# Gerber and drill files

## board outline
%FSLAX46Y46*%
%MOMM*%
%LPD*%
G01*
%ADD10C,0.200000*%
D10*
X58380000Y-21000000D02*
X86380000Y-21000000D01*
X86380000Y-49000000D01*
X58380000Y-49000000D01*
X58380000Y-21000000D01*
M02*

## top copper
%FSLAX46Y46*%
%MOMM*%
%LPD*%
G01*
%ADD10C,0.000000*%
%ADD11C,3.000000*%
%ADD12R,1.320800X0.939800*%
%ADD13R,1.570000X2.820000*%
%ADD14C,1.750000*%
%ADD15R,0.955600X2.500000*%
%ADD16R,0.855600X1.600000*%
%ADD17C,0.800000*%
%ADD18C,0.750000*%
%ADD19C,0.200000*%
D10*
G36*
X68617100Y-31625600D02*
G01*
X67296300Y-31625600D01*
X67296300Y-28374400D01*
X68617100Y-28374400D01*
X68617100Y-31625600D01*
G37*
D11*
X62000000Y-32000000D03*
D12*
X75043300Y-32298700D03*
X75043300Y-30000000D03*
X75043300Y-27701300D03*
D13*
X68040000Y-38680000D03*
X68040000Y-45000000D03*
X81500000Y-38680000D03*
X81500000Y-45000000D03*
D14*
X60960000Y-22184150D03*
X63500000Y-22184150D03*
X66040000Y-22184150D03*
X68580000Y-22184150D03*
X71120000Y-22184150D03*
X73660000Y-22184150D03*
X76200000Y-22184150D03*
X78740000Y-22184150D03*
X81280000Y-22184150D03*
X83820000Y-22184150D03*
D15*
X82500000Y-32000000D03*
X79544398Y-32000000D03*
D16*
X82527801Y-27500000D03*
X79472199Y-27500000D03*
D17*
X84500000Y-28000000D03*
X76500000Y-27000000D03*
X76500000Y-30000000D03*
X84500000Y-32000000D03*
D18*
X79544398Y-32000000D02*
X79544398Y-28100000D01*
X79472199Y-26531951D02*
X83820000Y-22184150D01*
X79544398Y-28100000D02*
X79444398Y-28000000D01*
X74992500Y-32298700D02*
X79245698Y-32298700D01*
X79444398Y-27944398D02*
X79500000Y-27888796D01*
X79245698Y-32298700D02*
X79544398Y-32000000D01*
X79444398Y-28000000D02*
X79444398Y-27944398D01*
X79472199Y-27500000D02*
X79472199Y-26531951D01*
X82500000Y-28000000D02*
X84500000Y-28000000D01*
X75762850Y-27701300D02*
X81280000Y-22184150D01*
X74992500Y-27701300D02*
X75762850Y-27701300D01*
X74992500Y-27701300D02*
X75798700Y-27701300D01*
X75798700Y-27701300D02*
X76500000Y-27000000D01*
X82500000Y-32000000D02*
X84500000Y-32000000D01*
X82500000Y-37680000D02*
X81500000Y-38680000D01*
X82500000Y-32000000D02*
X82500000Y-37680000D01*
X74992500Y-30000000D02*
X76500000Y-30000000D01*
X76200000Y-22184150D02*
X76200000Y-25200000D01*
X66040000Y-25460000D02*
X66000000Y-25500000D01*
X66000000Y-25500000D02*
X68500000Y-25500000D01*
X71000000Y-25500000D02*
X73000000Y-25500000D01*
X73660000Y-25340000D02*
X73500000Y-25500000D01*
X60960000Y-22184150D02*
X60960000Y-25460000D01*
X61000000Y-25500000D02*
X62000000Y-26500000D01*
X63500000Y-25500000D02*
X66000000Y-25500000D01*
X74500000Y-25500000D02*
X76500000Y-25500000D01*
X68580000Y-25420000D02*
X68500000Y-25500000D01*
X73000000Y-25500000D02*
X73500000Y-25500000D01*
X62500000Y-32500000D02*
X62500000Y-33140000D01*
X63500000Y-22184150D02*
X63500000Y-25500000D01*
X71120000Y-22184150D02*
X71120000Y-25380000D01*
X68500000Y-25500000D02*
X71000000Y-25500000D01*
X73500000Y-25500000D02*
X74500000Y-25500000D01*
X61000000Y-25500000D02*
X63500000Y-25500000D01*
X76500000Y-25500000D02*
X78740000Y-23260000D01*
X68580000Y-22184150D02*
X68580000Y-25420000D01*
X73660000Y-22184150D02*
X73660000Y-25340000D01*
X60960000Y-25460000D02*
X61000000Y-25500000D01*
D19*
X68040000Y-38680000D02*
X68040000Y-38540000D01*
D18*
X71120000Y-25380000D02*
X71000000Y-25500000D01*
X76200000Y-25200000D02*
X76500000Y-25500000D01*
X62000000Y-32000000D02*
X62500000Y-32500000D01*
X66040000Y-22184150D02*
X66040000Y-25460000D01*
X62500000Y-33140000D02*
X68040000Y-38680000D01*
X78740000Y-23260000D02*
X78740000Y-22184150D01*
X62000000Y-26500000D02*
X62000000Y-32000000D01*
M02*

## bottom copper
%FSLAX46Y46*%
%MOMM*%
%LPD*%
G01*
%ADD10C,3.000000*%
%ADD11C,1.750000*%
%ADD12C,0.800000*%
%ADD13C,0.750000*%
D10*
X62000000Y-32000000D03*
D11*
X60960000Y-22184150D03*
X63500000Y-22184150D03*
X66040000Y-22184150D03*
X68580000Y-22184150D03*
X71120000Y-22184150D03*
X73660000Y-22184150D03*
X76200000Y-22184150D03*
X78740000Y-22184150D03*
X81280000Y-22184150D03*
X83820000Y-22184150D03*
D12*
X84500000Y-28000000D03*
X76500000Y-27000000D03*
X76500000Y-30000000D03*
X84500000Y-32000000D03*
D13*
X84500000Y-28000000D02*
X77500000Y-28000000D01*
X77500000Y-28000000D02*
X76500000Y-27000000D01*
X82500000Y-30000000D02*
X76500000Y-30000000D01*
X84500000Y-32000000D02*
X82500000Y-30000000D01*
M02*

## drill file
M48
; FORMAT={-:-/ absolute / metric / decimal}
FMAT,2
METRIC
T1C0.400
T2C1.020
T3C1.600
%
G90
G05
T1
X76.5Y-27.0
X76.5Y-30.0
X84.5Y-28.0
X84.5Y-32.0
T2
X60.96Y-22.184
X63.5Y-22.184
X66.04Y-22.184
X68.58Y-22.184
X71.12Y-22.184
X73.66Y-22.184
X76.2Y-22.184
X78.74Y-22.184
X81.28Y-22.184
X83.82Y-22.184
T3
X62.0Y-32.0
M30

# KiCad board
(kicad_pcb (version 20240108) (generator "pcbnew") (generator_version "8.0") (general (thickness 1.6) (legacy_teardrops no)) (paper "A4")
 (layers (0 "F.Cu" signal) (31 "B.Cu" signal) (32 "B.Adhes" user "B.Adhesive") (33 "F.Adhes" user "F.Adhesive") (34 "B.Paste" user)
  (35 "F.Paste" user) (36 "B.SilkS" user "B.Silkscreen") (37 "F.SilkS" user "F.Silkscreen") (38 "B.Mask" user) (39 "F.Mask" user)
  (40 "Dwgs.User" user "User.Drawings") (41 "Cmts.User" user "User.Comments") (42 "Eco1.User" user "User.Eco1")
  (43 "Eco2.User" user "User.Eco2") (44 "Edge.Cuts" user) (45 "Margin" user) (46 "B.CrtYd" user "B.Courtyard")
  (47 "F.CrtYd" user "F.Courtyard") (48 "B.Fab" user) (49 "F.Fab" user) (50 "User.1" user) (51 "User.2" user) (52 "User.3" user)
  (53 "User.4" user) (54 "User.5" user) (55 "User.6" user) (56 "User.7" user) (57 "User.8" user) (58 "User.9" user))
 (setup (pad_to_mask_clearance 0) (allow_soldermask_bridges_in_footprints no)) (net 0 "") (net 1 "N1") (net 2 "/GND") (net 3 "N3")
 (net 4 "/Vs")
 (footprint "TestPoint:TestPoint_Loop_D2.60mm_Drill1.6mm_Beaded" (layer "F.Cu") (at 62 32)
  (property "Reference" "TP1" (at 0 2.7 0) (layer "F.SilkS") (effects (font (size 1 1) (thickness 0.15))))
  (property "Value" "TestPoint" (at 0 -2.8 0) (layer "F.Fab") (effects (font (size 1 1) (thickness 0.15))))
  (pad "1" thru_hole circle (at 0 0) (size 3 3) (drill 1.6) (layers "*.Cu" "*.Mask") (remove_unused_layers no) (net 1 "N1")))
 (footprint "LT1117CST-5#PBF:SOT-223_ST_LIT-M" (layer "F.Cu") (at 71.5 30 90)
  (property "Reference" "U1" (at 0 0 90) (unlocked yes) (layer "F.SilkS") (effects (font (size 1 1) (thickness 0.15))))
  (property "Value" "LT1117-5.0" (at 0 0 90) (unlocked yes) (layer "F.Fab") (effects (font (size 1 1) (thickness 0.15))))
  (fp_poly
   (pts (xy 1.6256 -4.2037) (xy -1.6256 -4.2037) (xy -1.6256 -2.8829) (xy 1.6256 -2.8829)) (stroke (width 0) (type solid)) (fill solid)
   (layer "F.Cu"))
  (pad "1" smd rect (at -2.2987 3.5433 90) (size 0.9398 1.3208) (layers "F.Cu" "F.Paste" "F.Mask") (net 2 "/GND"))
  (pad "2" smd rect (at 0 3.5433 90) (size 0.9398 1.3208) (layers "F.Cu" "F.Paste" "F.Mask") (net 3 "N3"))
  (pad "3" smd rect (at 2.2987 3.5433 90) (size 0.9398 1.3208) (layers "F.Cu" "F.Paste" "F.Mask") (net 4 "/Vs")))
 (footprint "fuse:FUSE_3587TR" (layer "F.Cu") (at 74.77 41.84)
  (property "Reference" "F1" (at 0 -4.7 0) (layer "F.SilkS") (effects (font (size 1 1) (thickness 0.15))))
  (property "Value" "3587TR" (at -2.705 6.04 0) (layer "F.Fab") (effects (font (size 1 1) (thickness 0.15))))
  (pad "1_1" smd rect (at -6.73 -3.16) (size 1.57 2.82) (layers "F.Cu" "F.Paste" "F.Mask") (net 1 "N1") (solder_mask_margin 0.102))
  (pad "1_2" smd rect (at -6.73 3.16) (size 1.57 2.82) (layers "F.Cu" "F.Paste" "F.Mask") (solder_mask_margin 0.102))
  (pad "2_1" smd rect (at 6.73 -3.16) (size 1.57 2.82) (layers "F.Cu" "F.Paste" "F.Mask") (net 3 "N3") (solder_mask_margin 0.102))
  (pad "2_2" smd rect (at 6.73 3.16) (size 1.57 2.82) (layers "F.Cu" "F.Paste" "F.Mask") (solder_mask_margin 0.102)))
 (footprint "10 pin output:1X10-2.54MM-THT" (layer "F.Cu") (at 60.96 22.18415)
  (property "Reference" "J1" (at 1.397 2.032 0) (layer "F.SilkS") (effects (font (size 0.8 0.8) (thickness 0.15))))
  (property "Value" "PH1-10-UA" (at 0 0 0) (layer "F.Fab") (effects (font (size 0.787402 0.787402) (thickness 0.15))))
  (pad "1" thru_hole circle (at 0 0) (size 1.75 1.75) (drill 1.02) (layers "*.Cu" "*.Mask") (remove_unused_layers no) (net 1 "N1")
   (solder_mask_margin 0.102))
  (pad "2" thru_hole circle (at 2.54 0) (size 1.75 1.75) (drill 1.02) (layers "*.Cu" "*.Mask") (remove_unused_layers no) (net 1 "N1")
   (solder_mask_margin 0.102))
  (pad "3" thru_hole circle (at 5.08 0) (size 1.75 1.75) (drill 1.02) (layers "*.Cu" "*.Mask") (remove_unused_layers no) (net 1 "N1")
   (solder_mask_margin 0.102))
  (pad "4" thru_hole circle (at 7.62 0) (size 1.75 1.75) (drill 1.02) (layers "*.Cu" "*.Mask") (remove_unused_layers no) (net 1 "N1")
   (solder_mask_margin 0.102))
  (pad "5" thru_hole circle (at 10.16 0) (size 1.75 1.75) (drill 1.02) (layers "*.Cu" "*.Mask") (remove_unused_layers no) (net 1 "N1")
   (solder_mask_margin 0.102))
  (pad "6" thru_hole circle (at 12.7 0) (size 1.75 1.75) (drill 1.02) (layers "*.Cu" "*.Mask") (remove_unused_layers no) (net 1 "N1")
   (solder_mask_margin 0.102))
  (pad "7" thru_hole circle (at 15.24 0) (size 1.75 1.75) (drill 1.02) (layers "*.Cu" "*.Mask") (remove_unused_layers no) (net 1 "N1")
   (solder_mask_margin 0.102))
  (pad "8" thru_hole circle (at 17.78 0) (size 1.75 1.75) (drill 1.02) (layers "*.Cu" "*.Mask") (remove_unused_layers no) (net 1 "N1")
   (solder_mask_margin 0.102))
  (pad "9" thru_hole circle (at 20.32 0) (size 1.75 1.75) (drill 1.02) (layers "*.Cu" "*.Mask") (remove_unused_layers no) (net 4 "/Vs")
   (solder_mask_margin 0.102))
  (pad "10" thru_hole circle (at 22.86 0) (size 1.75 1.75) (drill 1.02) (layers "*.Cu" "*.Mask") (remove_unused_layers no) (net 2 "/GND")
   (solder_mask_margin 0.102)))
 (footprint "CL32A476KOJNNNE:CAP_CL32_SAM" (layer "F.Cu") (at 81.022199 32 180)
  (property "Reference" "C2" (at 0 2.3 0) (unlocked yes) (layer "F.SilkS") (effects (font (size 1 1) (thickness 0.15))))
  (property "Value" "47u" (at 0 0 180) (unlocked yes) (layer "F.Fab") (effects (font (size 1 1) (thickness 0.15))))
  (pad "1" smd rect (at -1.477801 0 180) (size 0.9556 2.5) (layers "F.Cu" "F.Paste" "F.Mask") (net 3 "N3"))
  (pad "2" smd rect (at 1.477801 0 180) (size 0.9556 2.5) (layers "F.Cu" "F.Paste" "F.Mask") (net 2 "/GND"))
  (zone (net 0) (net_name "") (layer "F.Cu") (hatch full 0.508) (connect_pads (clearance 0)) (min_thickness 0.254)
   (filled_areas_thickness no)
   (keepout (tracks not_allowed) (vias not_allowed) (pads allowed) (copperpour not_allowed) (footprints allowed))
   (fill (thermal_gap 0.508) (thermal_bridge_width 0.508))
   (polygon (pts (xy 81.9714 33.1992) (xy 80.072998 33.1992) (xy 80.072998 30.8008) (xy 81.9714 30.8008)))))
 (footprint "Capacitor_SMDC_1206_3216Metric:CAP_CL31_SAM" (layer "F.Cu") (at 81 27.5 180)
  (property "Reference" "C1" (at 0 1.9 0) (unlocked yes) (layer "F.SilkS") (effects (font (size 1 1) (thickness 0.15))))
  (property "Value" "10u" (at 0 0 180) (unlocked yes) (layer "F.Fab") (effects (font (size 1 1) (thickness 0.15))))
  (pad "1" smd rect (at -1.527801 0 180) (size 0.8556 1.6) (layers "F.Cu" "F.Paste" "F.Mask") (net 4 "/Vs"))
  (pad "2" smd rect (at 1.527801 0 180) (size 0.8556 1.6) (layers "F.Cu" "F.Paste" "F.Mask") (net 2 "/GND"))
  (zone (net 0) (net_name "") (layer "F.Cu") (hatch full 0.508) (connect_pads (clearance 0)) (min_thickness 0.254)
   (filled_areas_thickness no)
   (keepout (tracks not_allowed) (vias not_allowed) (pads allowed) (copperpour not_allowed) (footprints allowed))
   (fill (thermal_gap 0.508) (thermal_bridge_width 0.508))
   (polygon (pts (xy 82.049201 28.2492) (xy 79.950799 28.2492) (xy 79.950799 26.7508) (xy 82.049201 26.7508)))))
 (gr_rect (start 58.38 21) (end 86.38 49) (stroke (width 0.2) (type default)) (fill none) (layer "Edge.Cuts"))
 (segment (start 79.544398 32) (end 79.544398 28.1) (width 0.75) (layer "F.Cu") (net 2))
 (segment (start 79.472199 26.531951) (end 83.82 22.18415) (width 0.75) (layer "F.Cu") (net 2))
 (segment (start 79.544398 28.1) (end 79.444398 28) (width 0.75) (layer "F.Cu") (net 2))
 (segment (start 74.9925 32.2987) (end 79.245698 32.2987) (width 0.75) (layer "F.Cu") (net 2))
 (segment (start 79.444398 27.944398) (end 79.5 27.888796) (width 0.75) (layer "F.Cu") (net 2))
 (segment (start 79.245698 32.2987) (end 79.544398 32) (width 0.75) (layer "F.Cu") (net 2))
 (segment (start 79.444398 28) (end 79.444398 27.944398) (width 0.75) (layer "F.Cu") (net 2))
 (segment (start 79.472199 27.5) (end 79.472199 26.531951) (width 0.75) (layer "F.Cu") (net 2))
 (segment (start 82.5 28) (end 84.5 28) (width 0.75) (layer "F.Cu") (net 4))
 (segment (start 75.76285 27.7013) (end 81.28 22.18415) (width 0.75) (layer "F.Cu") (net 4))
 (segment (start 74.9925 27.7013) (end 75.76285 27.7013) (width 0.75) (layer "F.Cu") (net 4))
 (segment (start 74.9925 27.7013) (end 75.7987 27.7013) (width 0.75) (layer "F.Cu") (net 4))
 (segment (start 75.7987 27.7013) (end 76.5 27) (width 0.75) (layer "F.Cu") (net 4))
 (via (at 84.5 28) (size 0.8) (drill 0.4) (layers "F.Cu" "B.Cu") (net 4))
 (via (at 76.5 27) (size 0.8) (drill 0.4) (layers "F.Cu" "B.Cu") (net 4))
 (segment (start 84.5 28) (end 77.5 28) (width 0.75) (layer "B.Cu") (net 4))
 (segment (start 77.5 28) (end 76.5 27) (width 0.75) (layer "B.Cu") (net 4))
 (segment (start 82.5 32) (end 84.5 32) (width 0.75) (layer "F.Cu") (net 3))
 (segment (start 82.5 37.68) (end 81.5 38.68) (width 0.75) (layer "F.Cu") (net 3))
 (segment (start 82.5 32) (end 82.5 37.68) (width 0.75) (layer "F.Cu") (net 3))
 (segment (start 74.9925 30) (end 76.5 30) (width 0.75) (layer "F.Cu") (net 3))
 (via (at 76.5 30) (size 0.8) (drill 0.4) (layers "F.Cu" "B.Cu") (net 3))
 (via (at 84.5 32) (size 0.8) (drill 0.4) (layers "F.Cu" "B.Cu") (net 3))
 (segment (start 82.5 30) (end 76.5 30) (width 0.75) (layer "B.Cu") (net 3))
 (segment (start 84.5 32) (end 82.5 30) (width 0.75) (layer "B.Cu") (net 3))
 (segment (start 76.2 22.18415) (end 76.2 25.2) (width 0.75) (layer "F.Cu") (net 1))
 (segment (start 66.04 25.46) (end 66 25.5) (width 0.75) (layer "F.Cu") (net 1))
 (segment (start 66 25.5) (end 68.5 25.5) (width 0.75) (layer "F.Cu") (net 1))
 (segment (start 71 25.5) (end 73 25.5) (width 0.75) (layer "F.Cu") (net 1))
 (segment (start 73.66 25.34) (end 73.5 25.5) (width 0.75) (layer "F.Cu") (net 1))
 (segment (start 60.96 22.18415) (end 60.96 25.46) (width 0.75) (layer "F.Cu") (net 1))
 (segment (start 61 25.5) (end 62 26.5) (width 0.75) (layer "F.Cu") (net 1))
 (segment (start 63.5 25.5) (end 66 25.5) (width 0.75) (layer "F.Cu") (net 1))
 (segment (start 74.5 25.5) (end 76.5 25.5) (width 0.75) (layer "F.Cu") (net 1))
 (segment (start 68.58 25.42) (end 68.5 25.5) (width 0.75) (layer "F.Cu") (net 1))
 (segment (start 73 25.5) (end 73.5 25.5) (width 0.75) (layer "F.Cu") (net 1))
 (segment (start 62.5 32.5) (end 62.5 33.14) (width 0.75) (layer "F.Cu") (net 1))
 (segment (start 63.5 22.18415) (end 63.5 25.5) (width 0.75) (layer "F.Cu") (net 1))
 (segment (start 71.12 22.18415) (end 71.12 25.38) (width 0.75) (layer "F.Cu") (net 1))
 (segment (start 68.5 25.5) (end 71 25.5) (width 0.75) (layer "F.Cu") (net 1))
 (segment (start 73.5 25.5) (end 74.5 25.5) (width 0.75) (layer "F.Cu") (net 1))
 (segment (start 61 25.5) (end 63.5 25.5) (width 0.75) (layer "F.Cu") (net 1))
 (segment (start 76.5 25.5) (end 78.74 23.26) (width 0.75) (layer "F.Cu") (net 1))
 (segment (start 68.58 22.18415) (end 68.58 25.42) (width 0.75) (layer "F.Cu") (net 1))
 (segment (start 73.66 22.18415) (end 73.66 25.34) (width 0.75) (layer "F.Cu") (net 1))
 (segment (start 60.96 25.46) (end 61 25.5) (width 0.75) (layer "F.Cu") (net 1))
 (segment (start 68.04 38.68) (end 68.04 38.54) (width 0.2) (layer "F.Cu") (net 1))
 (segment (start 71.12 25.38) (end 71 25.5) (width 0.75) (layer "F.Cu") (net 1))
 (segment (start 76.2 25.2) (end 76.5 25.5) (width 0.75) (layer "F.Cu") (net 1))
 (segment (start 62 32) (end 62.5 32.5) (width 0.75) (layer "F.Cu") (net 1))
 (segment (start 66.04 22.18415) (end 66.04 25.46) (width 0.75) (layer "F.Cu") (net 1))
 (segment (start 62.5 33.14) (end 68.04 38.68) (width 0.75) (layer "F.Cu") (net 1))
 (segment (start 78.74 23.26) (end 78.74 22.18415) (width 0.75) (layer "F.Cu") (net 1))
 (segment (start 62 26.5) (end 62 32) (width 0.75) (layer "F.Cu") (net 1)))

